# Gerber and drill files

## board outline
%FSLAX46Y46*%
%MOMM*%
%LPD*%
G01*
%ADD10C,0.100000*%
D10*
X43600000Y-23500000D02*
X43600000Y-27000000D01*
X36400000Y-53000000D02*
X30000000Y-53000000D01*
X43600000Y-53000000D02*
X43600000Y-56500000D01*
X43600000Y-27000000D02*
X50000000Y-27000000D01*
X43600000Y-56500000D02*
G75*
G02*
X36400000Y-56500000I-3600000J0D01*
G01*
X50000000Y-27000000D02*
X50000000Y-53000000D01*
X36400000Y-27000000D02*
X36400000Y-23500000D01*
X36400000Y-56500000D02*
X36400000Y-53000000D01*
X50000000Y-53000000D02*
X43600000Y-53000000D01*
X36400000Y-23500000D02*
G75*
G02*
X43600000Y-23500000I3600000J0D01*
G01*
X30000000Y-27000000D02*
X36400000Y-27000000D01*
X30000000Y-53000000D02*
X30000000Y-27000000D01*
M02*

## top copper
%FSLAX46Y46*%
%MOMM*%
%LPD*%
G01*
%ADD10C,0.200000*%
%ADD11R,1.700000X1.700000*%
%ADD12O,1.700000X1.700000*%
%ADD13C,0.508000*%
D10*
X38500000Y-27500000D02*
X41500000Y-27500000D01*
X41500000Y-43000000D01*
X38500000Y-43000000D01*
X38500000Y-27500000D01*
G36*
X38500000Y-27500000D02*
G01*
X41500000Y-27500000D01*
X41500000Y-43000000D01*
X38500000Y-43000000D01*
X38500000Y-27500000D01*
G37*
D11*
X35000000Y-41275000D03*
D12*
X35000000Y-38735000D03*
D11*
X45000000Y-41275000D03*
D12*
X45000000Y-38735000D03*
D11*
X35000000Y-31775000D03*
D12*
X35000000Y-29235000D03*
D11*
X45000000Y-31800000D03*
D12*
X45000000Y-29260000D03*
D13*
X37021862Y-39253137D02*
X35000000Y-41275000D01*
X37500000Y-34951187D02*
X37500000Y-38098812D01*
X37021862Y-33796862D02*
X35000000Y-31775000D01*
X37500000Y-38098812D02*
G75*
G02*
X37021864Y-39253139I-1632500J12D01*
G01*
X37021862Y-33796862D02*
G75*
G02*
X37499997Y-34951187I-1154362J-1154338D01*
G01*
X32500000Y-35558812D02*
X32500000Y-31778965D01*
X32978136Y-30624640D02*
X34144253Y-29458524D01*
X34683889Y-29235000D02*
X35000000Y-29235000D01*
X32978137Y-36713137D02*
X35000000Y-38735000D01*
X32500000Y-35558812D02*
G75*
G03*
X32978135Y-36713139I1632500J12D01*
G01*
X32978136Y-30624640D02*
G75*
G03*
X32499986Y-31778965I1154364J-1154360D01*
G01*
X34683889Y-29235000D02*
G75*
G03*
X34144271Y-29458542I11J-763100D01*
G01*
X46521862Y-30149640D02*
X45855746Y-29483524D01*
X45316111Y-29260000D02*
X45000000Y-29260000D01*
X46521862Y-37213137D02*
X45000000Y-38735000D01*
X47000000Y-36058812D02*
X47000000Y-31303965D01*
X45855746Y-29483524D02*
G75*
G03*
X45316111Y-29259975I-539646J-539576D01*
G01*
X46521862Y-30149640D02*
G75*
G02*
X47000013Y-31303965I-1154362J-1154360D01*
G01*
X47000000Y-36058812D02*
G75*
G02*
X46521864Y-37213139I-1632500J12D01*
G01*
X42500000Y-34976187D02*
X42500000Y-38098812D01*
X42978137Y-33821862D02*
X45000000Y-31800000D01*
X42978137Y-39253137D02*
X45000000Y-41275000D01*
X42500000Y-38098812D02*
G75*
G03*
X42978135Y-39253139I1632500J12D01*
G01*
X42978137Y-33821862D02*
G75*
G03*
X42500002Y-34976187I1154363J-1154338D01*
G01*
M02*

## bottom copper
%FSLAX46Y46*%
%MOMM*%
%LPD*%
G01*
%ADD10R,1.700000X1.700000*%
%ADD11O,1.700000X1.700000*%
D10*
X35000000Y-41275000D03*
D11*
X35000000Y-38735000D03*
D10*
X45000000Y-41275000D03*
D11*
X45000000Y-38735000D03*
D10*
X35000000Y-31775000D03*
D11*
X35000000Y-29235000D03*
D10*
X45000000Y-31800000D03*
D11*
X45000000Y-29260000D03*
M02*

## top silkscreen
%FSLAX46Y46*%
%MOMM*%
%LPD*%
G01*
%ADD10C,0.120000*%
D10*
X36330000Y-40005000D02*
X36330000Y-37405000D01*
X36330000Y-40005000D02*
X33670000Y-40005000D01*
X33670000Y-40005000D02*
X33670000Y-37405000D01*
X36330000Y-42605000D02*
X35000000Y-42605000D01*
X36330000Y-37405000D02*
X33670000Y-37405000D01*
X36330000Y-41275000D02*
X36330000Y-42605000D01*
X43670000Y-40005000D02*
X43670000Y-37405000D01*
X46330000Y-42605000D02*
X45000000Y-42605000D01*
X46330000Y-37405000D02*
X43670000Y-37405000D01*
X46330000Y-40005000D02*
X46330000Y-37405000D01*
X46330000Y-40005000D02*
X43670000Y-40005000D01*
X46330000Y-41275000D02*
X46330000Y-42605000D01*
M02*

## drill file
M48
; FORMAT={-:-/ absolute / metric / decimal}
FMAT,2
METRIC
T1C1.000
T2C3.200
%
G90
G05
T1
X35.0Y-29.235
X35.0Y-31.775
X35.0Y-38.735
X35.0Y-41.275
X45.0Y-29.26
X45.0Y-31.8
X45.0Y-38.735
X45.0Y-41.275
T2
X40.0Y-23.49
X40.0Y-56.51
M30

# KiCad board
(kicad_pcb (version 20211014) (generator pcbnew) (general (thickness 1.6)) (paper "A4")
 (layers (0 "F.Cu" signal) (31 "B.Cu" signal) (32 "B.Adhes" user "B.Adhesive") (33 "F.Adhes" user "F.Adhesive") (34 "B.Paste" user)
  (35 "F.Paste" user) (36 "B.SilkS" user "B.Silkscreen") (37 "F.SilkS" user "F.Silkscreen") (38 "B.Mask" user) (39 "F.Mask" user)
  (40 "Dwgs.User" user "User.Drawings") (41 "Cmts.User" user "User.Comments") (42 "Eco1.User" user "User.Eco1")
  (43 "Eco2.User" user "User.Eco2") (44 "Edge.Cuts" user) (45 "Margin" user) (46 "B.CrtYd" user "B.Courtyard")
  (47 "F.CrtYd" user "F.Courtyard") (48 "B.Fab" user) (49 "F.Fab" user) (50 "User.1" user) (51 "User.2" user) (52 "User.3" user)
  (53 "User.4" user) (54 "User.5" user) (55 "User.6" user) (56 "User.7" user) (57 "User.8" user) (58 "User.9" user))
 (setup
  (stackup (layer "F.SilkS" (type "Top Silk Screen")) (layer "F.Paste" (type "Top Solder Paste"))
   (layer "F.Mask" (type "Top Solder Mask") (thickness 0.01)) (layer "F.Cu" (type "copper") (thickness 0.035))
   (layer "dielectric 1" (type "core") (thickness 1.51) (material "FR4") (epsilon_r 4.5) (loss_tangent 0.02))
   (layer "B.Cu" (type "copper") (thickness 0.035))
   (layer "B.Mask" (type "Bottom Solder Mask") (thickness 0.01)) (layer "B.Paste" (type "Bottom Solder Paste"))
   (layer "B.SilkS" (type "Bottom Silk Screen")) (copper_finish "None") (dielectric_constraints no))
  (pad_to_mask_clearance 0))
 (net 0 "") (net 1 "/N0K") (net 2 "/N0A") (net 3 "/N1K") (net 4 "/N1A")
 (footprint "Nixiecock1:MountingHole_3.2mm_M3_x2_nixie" (layer "F.Cu") (at 40 40 90)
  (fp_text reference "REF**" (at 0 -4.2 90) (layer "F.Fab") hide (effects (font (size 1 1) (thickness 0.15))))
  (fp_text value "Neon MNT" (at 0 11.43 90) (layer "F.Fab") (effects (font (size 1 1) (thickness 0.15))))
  (pad "" np_thru_hole circle locked (at -16.51 0 90) (size 3.2 3.2) (drill 3.2) (layers *.Cu *.Mask))
  (pad "" np_thru_hole circle locked (at 16.51 0 90) (size 3.2 3.2) (drill 3.2) (layers *.Cu *.Mask)))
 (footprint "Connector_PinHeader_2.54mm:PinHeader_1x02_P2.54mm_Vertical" (layer "F.Cu") (at 35 41.275 180)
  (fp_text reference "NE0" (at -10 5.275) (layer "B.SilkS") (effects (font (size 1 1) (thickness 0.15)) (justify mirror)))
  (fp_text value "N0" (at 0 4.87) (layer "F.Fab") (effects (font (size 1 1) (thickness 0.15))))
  (fp_line (start -1.33 1.27) (end -1.33 3.87) (layer "F.SilkS") (width 0.12))
  (fp_line (start -1.33 1.27) (end 1.33 1.27) (layer "F.SilkS") (width 0.12))
  (fp_line (start 1.33 1.27) (end 1.33 3.87) (layer "F.SilkS") (width 0.12))
  (fp_line (start -1.33 -1.33) (end 0 -1.33) (layer "F.SilkS") (width 0.12))
  (fp_line (start -1.33 3.87) (end 1.33 3.87) (layer "F.SilkS") (width 0.12))
  (fp_line (start -1.33 0) (end -1.33 -1.33) (layer "F.SilkS") (width 0.12))
  (pad "1" thru_hole rect locked (at 0 0 180) (size 1.7 1.7) (drill 1) (layers *.Cu *.Mask) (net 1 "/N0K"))
  (pad "2" thru_hole oval locked (at 0 2.54 180) (size 1.7 1.7) (drill 1) (layers *.Cu *.Mask) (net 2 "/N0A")))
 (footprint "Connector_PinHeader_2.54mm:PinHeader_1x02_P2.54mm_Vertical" (layer "F.Cu") (at 45 41.275 180)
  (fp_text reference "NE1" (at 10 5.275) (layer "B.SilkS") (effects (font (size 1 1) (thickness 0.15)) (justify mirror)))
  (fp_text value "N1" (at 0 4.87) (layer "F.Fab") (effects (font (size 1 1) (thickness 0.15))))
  (fp_line (start 1.33 1.27) (end 1.33 3.87) (layer "F.SilkS") (width 0.12))
  (fp_line (start -1.33 -1.33) (end 0 -1.33) (layer "F.SilkS") (width 0.12))
  (fp_line (start -1.33 3.87) (end 1.33 3.87) (layer "F.SilkS") (width 0.12))
  (fp_line (start -1.33 1.27) (end -1.33 3.87) (layer "F.SilkS") (width 0.12))
  (fp_line (start -1.33 1.27) (end 1.33 1.27) (layer "F.SilkS") (width 0.12))
  (fp_line (start -1.33 0) (end -1.33 -1.33) (layer "F.SilkS") (width 0.12))
  (pad "1" thru_hole rect locked (at 0 0 180) (size 1.7 1.7) (drill 1) (layers *.Cu *.Mask) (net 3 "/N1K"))
  (pad "2" thru_hole oval locked (at 0 2.54 180) (size 1.7 1.7) (drill 1) (layers *.Cu *.Mask) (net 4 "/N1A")))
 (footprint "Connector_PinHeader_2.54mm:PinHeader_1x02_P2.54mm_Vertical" (layer "B.Cu") (at 35 31.775)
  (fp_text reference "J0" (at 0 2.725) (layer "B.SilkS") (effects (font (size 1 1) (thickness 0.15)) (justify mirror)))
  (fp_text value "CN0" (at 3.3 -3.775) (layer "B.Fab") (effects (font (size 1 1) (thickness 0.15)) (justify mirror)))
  (pad "1" thru_hole rect locked (at 0 0) (size 1.7 1.7) (drill 1) (layers *.Cu *.Mask) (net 1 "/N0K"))
  (pad "2" thru_hole oval locked (at 0 -2.54) (size 1.7 1.7) (drill 1) (layers *.Cu *.Mask) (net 2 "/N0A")))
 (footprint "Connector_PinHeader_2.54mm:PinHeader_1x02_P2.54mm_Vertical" (layer "B.Cu") (at 45 31.8)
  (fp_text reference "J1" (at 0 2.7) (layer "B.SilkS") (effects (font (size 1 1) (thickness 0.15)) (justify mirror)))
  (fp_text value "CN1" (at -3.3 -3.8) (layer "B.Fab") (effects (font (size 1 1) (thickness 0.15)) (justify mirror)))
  (pad "1" thru_hole rect locked (at 0 0) (size 1.7 1.7) (drill 1) (layers *.Cu *.Mask) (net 3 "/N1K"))
  (pad "2" thru_hole oval locked (at 0 -2.54) (size 1.7 1.7) (drill 1) (layers *.Cu *.Mask) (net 4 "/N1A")))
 (gr_rect (start 38.5 27.5) (end 41.5 43) (layer "F.Cu") (width 0.2) (fill solid))
 (gr_line (start 43.6 23.5) (end 43.6 27) (layer "Edge.Cuts") (width 0.1))
 (gr_line (start 36.4 53) (end 30 53) (layer "Edge.Cuts") (width 0.1))
 (gr_line (start 43.6 53) (end 43.6 56.5) (layer "Edge.Cuts") (width 0.1))
 (gr_line (start 43.6 27) (end 50 27) (layer "Edge.Cuts") (width 0.1))
 (gr_arc (start 43.6 56.5) (mid 40 60.1) (end 36.4 56.5) (layer "Edge.Cuts") (width 0.1))
 (gr_line (start 50 27) (end 50 53) (layer "Edge.Cuts") (width 0.1))
 (gr_line (start 36.4 27) (end 36.4 23.5) (layer "Edge.Cuts") (width 0.1))
 (gr_line (start 36.4 56.5) (end 36.4 53) (layer "Edge.Cuts") (width 0.1))
 (gr_line (start 50 53) (end 43.6 53) (layer "Edge.Cuts") (width 0.1))
 (gr_arc (start 36.4 23.5) (mid 40 19.9) (end 43.6 23.5) (layer "Edge.Cuts") (width 0.1))
 (gr_line (start 30 27) (end 36.4 27) (layer "Edge.Cuts") (width 0.1))
 (gr_line (start 30 53) (end 30 27) (layer "Edge.Cuts") (width 0.1))
 (segment (start 37.021862 39.253137) (end 35 41.275) (width 0.508) (layer "F.Cu") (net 1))
 (segment (start 37.5 34.951187) (end 37.5 38.098812) (width 0.508) (layer "F.Cu") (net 1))
 (segment (start 37.021862 33.796862) (end 35 31.775) (width 0.508) (layer "F.Cu") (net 1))
 (arc (start 37.5 38.098812) (mid 37.375735 38.723528) (end 37.021862 39.253137) (width 0.508) (layer "F.Cu") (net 1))
 (arc (start 37.021862 33.796862) (mid 37.375735 34.326471) (end 37.5 34.951187) (width 0.508) (layer "F.Cu") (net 1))
 (segment (start 32.5 35.558812) (end 32.5 31.778965) (width 0.508) (layer "F.Cu") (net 2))
 (segment (start 32.978136 30.62464) (end 34.144253 29.458524) (width 0.508) (layer "F.Cu") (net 2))
 (segment (start 34.683889 29.235) (end 35 29.235) (width 0.508) (layer "F.Cu") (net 2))
 (segment (start 32.978137 36.713137) (end 35 38.735) (width 0.508) (layer "F.Cu") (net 2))
 (arc (start 32.5 35.558812) (mid 32.624263 36.183528) (end 32.978137 36.713137) (width 0.508) (layer "F.Cu") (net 2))
 (arc (start 32.978136 30.62464) (mid 32.624263 31.154249) (end 32.5 31.778965) (width 0.508) (layer "F.Cu") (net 2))
 (arc (start 34.683889 29.235) (mid 34.39184 29.293091) (end 34.144253 29.458524) (width 0.508) (layer "F.Cu") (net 2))
 (segment (start 46.521862 30.14964) (end 45.855746 29.483524) (width 0.508) (layer "F.Cu") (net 4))
 (segment (start 45.316111 29.26) (end 45 29.26) (width 0.508) (layer "F.Cu") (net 4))
 (segment (start 46.521862 37.213137) (end 45 38.735) (width 0.508) (layer "F.Cu") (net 4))
 (segment (start 47 36.058812) (end 47 31.303965) (width 0.508) (layer "F.Cu") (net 4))
 (arc (start 45.855746 29.483524) (mid 45.608159 29.318091) (end 45.316111 29.26) (width 0.508) (layer "F.Cu") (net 4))
 (arc (start 46.521862 30.14964) (mid 46.875735 30.679249) (end 47 31.303965) (width 0.508) (layer "F.Cu") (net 4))
 (arc (start 47 36.058812) (mid 46.875735 36.683528) (end 46.521862 37.213137) (width 0.508) (layer "F.Cu") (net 4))
 (segment (start 42.5 34.976187) (end 42.5 38.098812) (width 0.508) (layer "F.Cu") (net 3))
 (segment (start 42.978137 33.821862) (end 45 31.8) (width 0.508) (layer "F.Cu") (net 3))
 (segment (start 42.978137 39.253137) (end 45 41.275) (width 0.508) (layer "F.Cu") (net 3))
 (arc (start 42.5 38.098812) (mid 42.624263 38.723528) (end 42.978137 39.253137) (width 0.508) (layer "F.Cu") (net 3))
 (arc (start 42.978137 33.821862) (mid 42.624263 34.351471) (end 42.5 34.976187) (width 0.508) (layer "F.Cu") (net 3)))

